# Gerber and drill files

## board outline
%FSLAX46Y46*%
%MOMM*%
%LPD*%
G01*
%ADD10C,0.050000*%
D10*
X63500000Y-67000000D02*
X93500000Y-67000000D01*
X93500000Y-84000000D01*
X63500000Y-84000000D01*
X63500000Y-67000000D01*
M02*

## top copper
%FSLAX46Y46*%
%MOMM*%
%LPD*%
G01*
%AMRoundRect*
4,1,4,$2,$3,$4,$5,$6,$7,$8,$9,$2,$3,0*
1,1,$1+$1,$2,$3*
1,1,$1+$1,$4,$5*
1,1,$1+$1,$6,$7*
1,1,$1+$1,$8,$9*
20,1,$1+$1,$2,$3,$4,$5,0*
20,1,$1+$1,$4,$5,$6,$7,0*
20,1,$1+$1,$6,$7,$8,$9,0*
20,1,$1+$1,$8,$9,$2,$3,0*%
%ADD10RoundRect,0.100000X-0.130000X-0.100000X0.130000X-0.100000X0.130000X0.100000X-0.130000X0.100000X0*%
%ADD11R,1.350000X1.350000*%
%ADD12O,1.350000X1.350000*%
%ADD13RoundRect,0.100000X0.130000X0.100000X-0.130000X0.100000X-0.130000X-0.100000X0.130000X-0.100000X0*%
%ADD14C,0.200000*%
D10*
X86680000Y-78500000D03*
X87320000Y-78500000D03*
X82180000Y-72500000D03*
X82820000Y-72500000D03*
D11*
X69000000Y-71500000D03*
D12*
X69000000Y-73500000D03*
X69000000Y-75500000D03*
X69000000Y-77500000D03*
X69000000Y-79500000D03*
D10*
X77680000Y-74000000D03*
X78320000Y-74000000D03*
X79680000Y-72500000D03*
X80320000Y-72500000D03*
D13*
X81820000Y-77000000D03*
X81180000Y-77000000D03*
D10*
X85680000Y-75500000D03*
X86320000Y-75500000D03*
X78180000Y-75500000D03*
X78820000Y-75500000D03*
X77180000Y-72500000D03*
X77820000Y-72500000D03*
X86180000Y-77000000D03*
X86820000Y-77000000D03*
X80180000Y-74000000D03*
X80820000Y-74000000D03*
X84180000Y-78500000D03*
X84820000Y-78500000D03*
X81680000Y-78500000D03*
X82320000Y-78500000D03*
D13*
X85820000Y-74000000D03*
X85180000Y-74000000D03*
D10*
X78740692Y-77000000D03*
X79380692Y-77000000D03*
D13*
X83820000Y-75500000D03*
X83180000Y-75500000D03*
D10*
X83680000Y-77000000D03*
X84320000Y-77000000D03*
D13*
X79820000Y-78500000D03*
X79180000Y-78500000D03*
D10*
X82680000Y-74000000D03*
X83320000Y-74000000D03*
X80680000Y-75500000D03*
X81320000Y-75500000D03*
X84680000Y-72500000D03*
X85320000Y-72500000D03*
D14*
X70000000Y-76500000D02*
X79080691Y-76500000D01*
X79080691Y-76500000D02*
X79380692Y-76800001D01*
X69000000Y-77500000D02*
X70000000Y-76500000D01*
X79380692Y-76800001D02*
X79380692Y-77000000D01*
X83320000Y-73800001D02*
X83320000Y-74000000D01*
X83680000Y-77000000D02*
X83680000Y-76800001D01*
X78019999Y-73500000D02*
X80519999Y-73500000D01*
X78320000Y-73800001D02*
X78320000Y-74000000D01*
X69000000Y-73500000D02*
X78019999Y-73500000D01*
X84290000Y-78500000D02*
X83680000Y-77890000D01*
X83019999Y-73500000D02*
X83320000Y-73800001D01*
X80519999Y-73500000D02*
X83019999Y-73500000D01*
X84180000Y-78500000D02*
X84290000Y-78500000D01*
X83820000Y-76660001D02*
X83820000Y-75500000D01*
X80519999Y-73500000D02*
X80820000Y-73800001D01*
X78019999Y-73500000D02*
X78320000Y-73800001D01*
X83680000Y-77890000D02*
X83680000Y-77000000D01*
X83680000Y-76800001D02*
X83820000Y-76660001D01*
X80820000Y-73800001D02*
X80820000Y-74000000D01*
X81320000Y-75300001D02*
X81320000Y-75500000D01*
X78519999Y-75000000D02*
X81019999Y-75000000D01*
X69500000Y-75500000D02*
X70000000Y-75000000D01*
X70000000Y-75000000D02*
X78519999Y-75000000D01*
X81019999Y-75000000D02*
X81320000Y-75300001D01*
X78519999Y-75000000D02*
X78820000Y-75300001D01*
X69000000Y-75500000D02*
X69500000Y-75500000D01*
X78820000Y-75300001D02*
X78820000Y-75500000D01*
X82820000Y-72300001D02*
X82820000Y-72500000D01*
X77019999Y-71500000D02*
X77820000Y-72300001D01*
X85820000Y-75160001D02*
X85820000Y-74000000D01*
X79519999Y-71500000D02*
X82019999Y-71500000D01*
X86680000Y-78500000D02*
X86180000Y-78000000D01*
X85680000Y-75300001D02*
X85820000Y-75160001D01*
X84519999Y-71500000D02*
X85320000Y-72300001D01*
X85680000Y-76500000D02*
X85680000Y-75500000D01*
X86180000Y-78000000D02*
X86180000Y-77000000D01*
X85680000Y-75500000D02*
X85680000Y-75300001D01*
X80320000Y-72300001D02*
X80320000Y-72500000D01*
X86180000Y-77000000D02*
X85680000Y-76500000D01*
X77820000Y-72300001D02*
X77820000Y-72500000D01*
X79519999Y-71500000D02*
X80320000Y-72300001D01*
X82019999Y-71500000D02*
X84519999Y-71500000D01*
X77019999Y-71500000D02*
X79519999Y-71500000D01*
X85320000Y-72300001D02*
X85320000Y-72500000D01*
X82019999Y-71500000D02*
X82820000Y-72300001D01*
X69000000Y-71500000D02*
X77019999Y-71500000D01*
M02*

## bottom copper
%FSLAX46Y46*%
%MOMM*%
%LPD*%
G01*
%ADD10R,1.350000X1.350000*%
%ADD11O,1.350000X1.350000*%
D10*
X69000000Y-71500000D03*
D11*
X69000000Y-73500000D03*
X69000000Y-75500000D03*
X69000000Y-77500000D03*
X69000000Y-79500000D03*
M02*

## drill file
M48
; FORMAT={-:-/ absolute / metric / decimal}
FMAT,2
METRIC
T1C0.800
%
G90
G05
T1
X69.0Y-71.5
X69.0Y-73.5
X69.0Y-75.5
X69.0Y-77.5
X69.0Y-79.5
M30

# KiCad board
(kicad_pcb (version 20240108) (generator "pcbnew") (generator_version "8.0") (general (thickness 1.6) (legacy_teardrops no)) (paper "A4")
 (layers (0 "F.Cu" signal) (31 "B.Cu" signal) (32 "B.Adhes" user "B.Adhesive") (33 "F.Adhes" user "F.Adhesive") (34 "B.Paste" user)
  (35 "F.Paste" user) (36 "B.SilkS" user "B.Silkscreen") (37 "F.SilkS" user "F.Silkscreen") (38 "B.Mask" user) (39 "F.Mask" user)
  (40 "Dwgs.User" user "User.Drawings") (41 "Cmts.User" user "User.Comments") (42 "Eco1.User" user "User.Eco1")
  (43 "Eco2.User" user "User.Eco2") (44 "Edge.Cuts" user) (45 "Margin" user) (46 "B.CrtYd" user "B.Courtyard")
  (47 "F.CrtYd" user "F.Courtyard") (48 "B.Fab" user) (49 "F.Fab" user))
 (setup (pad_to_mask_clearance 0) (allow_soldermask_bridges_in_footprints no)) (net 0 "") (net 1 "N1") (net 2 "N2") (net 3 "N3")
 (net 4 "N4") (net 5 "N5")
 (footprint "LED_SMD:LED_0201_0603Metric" (layer "F.Cu") (at 87 78.5)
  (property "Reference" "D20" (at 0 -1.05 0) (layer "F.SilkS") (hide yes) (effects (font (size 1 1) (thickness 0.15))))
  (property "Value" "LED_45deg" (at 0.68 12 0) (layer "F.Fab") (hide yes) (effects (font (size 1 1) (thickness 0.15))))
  (pad "" smd roundrect (at -0.345 0) (size 0.318 0.36) (layers "F.Paste") (roundrect_rratio 0.25))
  (pad "" smd roundrect (at 0.345 0) (size 0.318 0.36) (layers "F.Paste") (roundrect_rratio 0.25))
  (pad "1" smd roundrect (at -0.32 0) (size 0.46 0.4) (layers "F.Cu" "F.Mask") (roundrect_rratio 0.25) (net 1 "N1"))
  (pad "2" smd roundrect (at 0.32 0) (size 0.46 0.4) (layers "F.Cu" "F.Mask") (roundrect_rratio 0.25) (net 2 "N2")))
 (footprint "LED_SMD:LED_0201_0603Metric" (layer "F.Cu") (at 82.5 72.5)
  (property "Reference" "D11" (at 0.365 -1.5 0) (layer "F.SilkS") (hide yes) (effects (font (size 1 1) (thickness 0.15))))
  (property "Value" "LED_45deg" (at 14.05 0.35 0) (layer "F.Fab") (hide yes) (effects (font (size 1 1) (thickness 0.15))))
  (pad "" smd roundrect (at -0.345 0) (size 0.318 0.36) (layers "F.Paste") (roundrect_rratio 0.25))
  (pad "" smd roundrect (at 0.345 0) (size 0.318 0.36) (layers "F.Paste") (roundrect_rratio 0.25))
  (pad "1" smd roundrect (at -0.32 0) (size 0.46 0.4) (layers "F.Cu" "F.Mask") (roundrect_rratio 0.25) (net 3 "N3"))
  (pad "2" smd roundrect (at 0.32 0) (size 0.46 0.4) (layers "F.Cu" "F.Mask") (roundrect_rratio 0.25) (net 1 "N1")))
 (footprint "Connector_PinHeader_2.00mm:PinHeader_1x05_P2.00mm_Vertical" (layer "F.Cu") (at 69 71.5)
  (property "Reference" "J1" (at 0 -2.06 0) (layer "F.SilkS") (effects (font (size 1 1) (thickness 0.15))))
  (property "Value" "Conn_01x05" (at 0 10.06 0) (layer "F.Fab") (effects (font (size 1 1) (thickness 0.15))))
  (pad "1" thru_hole rect (at 0 0) (size 1.35 1.35) (drill 0.8) (layers "*.Cu" "*.Mask") (remove_unused_layers no) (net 1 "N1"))
  (pad "2" thru_hole oval (at 0 2) (size 1.35 1.35) (drill 0.8) (layers "*.Cu" "*.Mask") (remove_unused_layers no) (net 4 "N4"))
  (pad "3" thru_hole oval (at 0 4) (size 1.35 1.35) (drill 0.8) (layers "*.Cu" "*.Mask") (remove_unused_layers no) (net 3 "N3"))
  (pad "4" thru_hole oval (at 0 6) (size 1.35 1.35) (drill 0.8) (layers "*.Cu" "*.Mask") (remove_unused_layers no) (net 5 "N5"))
  (pad "5" thru_hole oval (at 0 8) (size 1.35 1.35) (drill 0.8) (layers "*.Cu" "*.Mask") (remove_unused_layers no) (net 2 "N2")))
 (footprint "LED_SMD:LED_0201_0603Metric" (layer "F.Cu") (at 78 74)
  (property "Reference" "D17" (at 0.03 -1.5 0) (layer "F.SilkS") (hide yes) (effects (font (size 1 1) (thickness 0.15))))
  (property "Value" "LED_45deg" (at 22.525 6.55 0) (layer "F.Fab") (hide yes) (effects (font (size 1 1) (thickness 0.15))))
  (pad "" smd roundrect (at -0.345 0) (size 0.318 0.36) (layers "F.Paste") (roundrect_rratio 0.25))
  (pad "" smd roundrect (at 0.345 0) (size 0.318 0.36) (layers "F.Paste") (roundrect_rratio 0.25))
  (pad "1" smd roundrect (at -0.32 0) (size 0.46 0.4) (layers "F.Cu" "F.Mask") (roundrect_rratio 0.25) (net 2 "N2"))
  (pad "2" smd roundrect (at 0.32 0) (size 0.46 0.4) (layers "F.Cu" "F.Mask") (roundrect_rratio 0.25) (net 4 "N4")))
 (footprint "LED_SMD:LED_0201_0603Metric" (layer "F.Cu") (at 80 72.5)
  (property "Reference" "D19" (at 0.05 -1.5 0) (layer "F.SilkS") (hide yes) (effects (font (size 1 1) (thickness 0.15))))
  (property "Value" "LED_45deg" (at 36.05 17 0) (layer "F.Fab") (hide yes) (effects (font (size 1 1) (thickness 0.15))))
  (pad "" smd roundrect (at -0.345 0) (size 0.318 0.36) (layers "F.Paste") (roundrect_rratio 0.25))
  (pad "" smd roundrect (at 0.345 0) (size 0.318 0.36) (layers "F.Paste") (roundrect_rratio 0.25))
  (pad "1" smd roundrect (at -0.32 0) (size 0.46 0.4) (layers "F.Cu" "F.Mask") (roundrect_rratio 0.25) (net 5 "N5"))
  (pad "2" smd roundrect (at 0.32 0) (size 0.46 0.4) (layers "F.Cu" "F.Mask") (roundrect_rratio 0.25) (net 1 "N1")))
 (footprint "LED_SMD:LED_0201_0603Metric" (layer "F.Cu") (at 81.5 77 180)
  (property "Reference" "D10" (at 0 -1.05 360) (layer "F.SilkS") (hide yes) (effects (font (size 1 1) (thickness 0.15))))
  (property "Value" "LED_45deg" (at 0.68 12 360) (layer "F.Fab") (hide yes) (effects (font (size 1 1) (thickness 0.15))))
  (pad "" smd roundrect (at -0.345 0 180) (size 0.318 0.36) (layers "F.Paste") (roundrect_rratio 0.25))
  (pad "" smd roundrect (at 0.345 0 180) (size 0.318 0.36) (layers "F.Paste") (roundrect_rratio 0.25))
  (pad "1" smd roundrect (at -0.32 0 180) (size 0.46 0.4) (layers "F.Cu" "F.Mask") (roundrect_rratio 0.25) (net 3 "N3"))
  (pad "2" smd roundrect (at 0.32 0 180) (size 0.46 0.4) (layers "F.Cu" "F.Mask") (roundrect_rratio 0.25) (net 5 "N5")))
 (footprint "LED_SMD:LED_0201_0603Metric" (layer "F.Cu") (at 86 75.5)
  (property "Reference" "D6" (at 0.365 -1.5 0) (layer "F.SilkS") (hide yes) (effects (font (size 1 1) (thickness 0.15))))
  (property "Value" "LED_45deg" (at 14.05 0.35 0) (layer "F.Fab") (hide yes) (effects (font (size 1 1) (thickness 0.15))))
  (pad "" smd roundrect (at -0.345 0) (size 0.318 0.36) (layers "F.Paste") (roundrect_rratio 0.25))
  (pad "" smd roundrect (at 0.345 0) (size 0.318 0.36) (layers "F.Paste") (roundrect_rratio 0.25))
  (pad "1" smd roundrect (at -0.32 0) (size 0.46 0.4) (layers "F.Cu" "F.Mask") (roundrect_rratio 0.25) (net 1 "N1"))
  (pad "2" smd roundrect (at 0.32 0) (size 0.46 0.4) (layers "F.Cu" "F.Mask") (roundrect_rratio 0.25) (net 3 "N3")))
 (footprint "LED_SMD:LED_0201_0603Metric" (layer "F.Cu") (at 78.5 75.5)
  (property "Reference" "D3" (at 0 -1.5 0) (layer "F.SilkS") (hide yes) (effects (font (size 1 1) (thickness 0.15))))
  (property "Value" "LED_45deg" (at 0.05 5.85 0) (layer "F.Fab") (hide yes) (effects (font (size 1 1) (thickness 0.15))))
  (pad "" smd roundrect (at -0.345 0) (size 0.318 0.36) (layers "F.Paste") (roundrect_rratio 0.25))
  (pad "" smd roundrect (at 0.345 0) (size 0.318 0.36) (layers "F.Paste") (roundrect_rratio 0.25))
  (pad "1" smd roundrect (at -0.32 0) (size 0.46 0.4) (layers "F.Cu" "F.Mask") (roundrect_rratio 0.25) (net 2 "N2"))
  (pad "2" smd roundrect (at 0.32 0) (size 0.46 0.4) (layers "F.Cu" "F.Mask") (roundrect_rratio 0.25) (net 3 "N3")))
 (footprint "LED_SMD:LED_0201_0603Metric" (layer "F.Cu") (at 77.5 72.5)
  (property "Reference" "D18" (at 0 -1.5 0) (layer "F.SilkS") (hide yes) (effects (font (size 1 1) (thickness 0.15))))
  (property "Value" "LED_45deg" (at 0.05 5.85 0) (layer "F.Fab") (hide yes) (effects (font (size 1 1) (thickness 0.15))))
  (pad "" smd roundrect (at -0.345 0) (size 0.318 0.36) (layers "F.Paste") (roundrect_rratio 0.25))
  (pad "" smd roundrect (at 0.345 0) (size 0.318 0.36) (layers "F.Paste") (roundrect_rratio 0.25))
  (pad "1" smd roundrect (at -0.32 0) (size 0.46 0.4) (layers "F.Cu" "F.Mask") (roundrect_rratio 0.25) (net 2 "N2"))
  (pad "2" smd roundrect (at 0.32 0) (size 0.46 0.4) (layers "F.Cu" "F.Mask") (roundrect_rratio 0.25) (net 1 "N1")))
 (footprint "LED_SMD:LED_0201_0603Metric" (layer "F.Cu") (at 86.5 77)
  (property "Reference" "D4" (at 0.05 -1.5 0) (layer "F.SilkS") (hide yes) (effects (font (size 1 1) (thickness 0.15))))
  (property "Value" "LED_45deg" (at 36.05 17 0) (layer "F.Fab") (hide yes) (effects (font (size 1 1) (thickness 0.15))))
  (pad "" smd roundrect (at -0.345 0) (size 0.318 0.36) (layers "F.Paste") (roundrect_rratio 0.25))
  (pad "" smd roundrect (at 0.345 0) (size 0.318 0.36) (layers "F.Paste") (roundrect_rratio 0.25))
  (pad "1" smd roundrect (at -0.32 0) (size 0.46 0.4) (layers "F.Cu" "F.Mask") (roundrect_rratio 0.25) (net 1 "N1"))
  (pad "2" smd roundrect (at 0.32 0) (size 0.46 0.4) (layers "F.Cu" "F.Mask") (roundrect_rratio 0.25) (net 5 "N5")))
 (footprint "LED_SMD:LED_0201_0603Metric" (layer "F.Cu") (at 80.5 74)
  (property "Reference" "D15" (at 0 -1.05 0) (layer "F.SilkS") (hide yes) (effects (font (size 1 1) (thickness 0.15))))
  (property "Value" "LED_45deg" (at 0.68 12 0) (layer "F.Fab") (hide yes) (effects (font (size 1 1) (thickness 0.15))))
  (pad "" smd roundrect (at -0.345 0) (size 0.318 0.36) (layers "F.Paste") (roundrect_rratio 0.25))
  (pad "" smd roundrect (at 0.345 0) (size 0.318 0.36) (layers "F.Paste") (roundrect_rratio 0.25))
  (pad "1" smd roundrect (at -0.32 0) (size 0.46 0.4) (layers "F.Cu" "F.Mask") (roundrect_rratio 0.25) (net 5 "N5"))
  (pad "2" smd roundrect (at 0.32 0) (size 0.46 0.4) (layers "F.Cu" "F.Mask") (roundrect_rratio 0.25) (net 4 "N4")))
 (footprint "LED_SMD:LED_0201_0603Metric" (layer "F.Cu") (at 84.5 78.5)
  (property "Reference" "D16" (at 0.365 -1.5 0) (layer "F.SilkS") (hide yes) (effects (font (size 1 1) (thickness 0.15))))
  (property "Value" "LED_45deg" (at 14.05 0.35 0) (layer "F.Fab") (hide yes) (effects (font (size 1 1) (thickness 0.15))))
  (pad "" smd roundrect (at -0.345 0) (size 0.318 0.36) (layers "F.Paste") (roundrect_rratio 0.25))
  (pad "" smd roundrect (at 0.345 0) (size 0.318 0.36) (layers "F.Paste") (roundrect_rratio 0.25))
  (pad "1" smd roundrect (at -0.32 0) (size 0.46 0.4) (layers "F.Cu" "F.Mask") (roundrect_rratio 0.25) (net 4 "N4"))
  (pad "2" smd roundrect (at 0.32 0) (size 0.46 0.4) (layers "F.Cu" "F.Mask") (roundrect_rratio 0.25) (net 2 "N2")))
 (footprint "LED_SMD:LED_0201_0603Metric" (layer "F.Cu") (at 82 78.5)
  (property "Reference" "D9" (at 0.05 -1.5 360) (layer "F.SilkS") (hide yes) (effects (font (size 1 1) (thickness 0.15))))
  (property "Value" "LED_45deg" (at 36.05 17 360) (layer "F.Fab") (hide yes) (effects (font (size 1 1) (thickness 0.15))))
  (pad "" smd roundrect (at -0.345 0) (size 0.318 0.36) (layers "F.Paste") (roundrect_rratio 0.25))
  (pad "" smd roundrect (at 0.345 0) (size 0.318 0.36) (layers "F.Paste") (roundrect_rratio 0.25))
  (pad "1" smd roundrect (at -0.32 0) (size 0.46 0.4) (layers "F.Cu" "F.Mask") (roundrect_rratio 0.25) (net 3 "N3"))
  (pad "2" smd roundrect (at 0.32 0) (size 0.46 0.4) (layers "F.Cu" "F.Mask") (roundrect_rratio 0.25) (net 2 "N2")))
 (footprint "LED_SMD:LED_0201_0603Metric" (layer "F.Cu") (at 85.5 74 180)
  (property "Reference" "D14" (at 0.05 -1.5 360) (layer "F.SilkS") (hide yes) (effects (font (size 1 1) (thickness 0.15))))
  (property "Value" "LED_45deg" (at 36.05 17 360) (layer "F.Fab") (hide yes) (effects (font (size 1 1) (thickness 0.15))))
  (pad "" smd roundrect (at -0.345 0 180) (size 0.318 0.36) (layers "F.Paste") (roundrect_rratio 0.25))
  (pad "" smd roundrect (at 0.345 0 180) (size 0.318 0.36) (layers "F.Paste") (roundrect_rratio 0.25))
  (pad "1" smd roundrect (at -0.32 0 180) (size 0.46 0.4) (layers "F.Cu" "F.Mask") (roundrect_rratio 0.25) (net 1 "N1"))
  (pad "2" smd roundrect (at 0.32 0 180) (size 0.46 0.4) (layers "F.Cu" "F.Mask") (roundrect_rratio 0.25) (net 4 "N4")))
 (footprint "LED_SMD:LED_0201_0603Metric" (layer "F.Cu") (at 79.060692 77)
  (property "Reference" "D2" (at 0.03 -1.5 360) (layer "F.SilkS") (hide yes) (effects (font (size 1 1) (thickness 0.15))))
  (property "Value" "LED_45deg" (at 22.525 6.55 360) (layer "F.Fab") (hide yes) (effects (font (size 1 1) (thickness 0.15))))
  (pad "" smd roundrect (at -0.345 0) (size 0.318 0.36) (layers "F.Paste") (roundrect_rratio 0.25))
  (pad "" smd roundrect (at 0.345 0) (size 0.318 0.36) (layers "F.Paste") (roundrect_rratio 0.25))
  (pad "1" smd roundrect (at -0.32 0) (size 0.46 0.4) (layers "F.Cu" "F.Mask") (roundrect_rratio 0.25) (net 2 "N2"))
  (pad "2" smd roundrect (at 0.32 0) (size 0.46 0.4) (layers "F.Cu" "F.Mask") (roundrect_rratio 0.25) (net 5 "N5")))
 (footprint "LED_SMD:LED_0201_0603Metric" (layer "F.Cu") (at 83.5 75.5 180)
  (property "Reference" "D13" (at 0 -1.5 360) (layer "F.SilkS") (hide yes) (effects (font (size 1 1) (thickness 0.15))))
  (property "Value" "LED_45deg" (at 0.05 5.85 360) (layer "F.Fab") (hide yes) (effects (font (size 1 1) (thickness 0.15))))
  (pad "" smd roundrect (at -0.345 0 180) (size 0.318 0.36) (layers "F.Paste") (roundrect_rratio 0.25))
  (pad "" smd roundrect (at 0.345 0 180) (size 0.318 0.36) (layers "F.Paste") (roundrect_rratio 0.25))
  (pad "1" smd roundrect (at -0.32 0 180) (size 0.46 0.4) (layers "F.Cu" "F.Mask") (roundrect_rratio 0.25) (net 4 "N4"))
  (pad "2" smd roundrect (at 0.32 0 180) (size 0.46 0.4) (layers "F.Cu" "F.Mask") (roundrect_rratio 0.25) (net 3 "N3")))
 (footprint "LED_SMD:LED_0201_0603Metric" (layer "F.Cu") (at 84 77)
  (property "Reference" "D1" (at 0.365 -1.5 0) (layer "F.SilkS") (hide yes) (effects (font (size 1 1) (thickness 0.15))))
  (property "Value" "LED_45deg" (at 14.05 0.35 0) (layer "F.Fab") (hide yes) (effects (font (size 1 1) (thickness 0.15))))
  (pad "" smd roundrect (at -0.345 0) (size 0.318 0.36) (layers "F.Paste") (roundrect_rratio 0.25))
  (pad "" smd roundrect (at 0.345 0) (size 0.318 0.36) (layers "F.Paste") (roundrect_rratio 0.25))
  (pad "1" smd roundrect (at -0.32 0) (size 0.46 0.4) (layers "F.Cu" "F.Mask") (roundrect_rratio 0.25) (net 4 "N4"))
  (pad "2" smd roundrect (at 0.32 0) (size 0.46 0.4) (layers "F.Cu" "F.Mask") (roundrect_rratio 0.25) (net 5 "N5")))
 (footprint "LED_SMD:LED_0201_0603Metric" (layer "F.Cu") (at 79.5 78.5 180)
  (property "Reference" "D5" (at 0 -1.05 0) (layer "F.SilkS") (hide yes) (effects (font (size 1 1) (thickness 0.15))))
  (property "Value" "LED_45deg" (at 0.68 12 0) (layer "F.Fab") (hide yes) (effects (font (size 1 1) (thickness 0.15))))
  (pad "" smd roundrect (at -0.345 0 180) (size 0.318 0.36) (layers "F.Paste") (roundrect_rratio 0.25))
  (pad "" smd roundrect (at 0.345 0 180) (size 0.318 0.36) (layers "F.Paste") (roundrect_rratio 0.25))
  (pad "1" smd roundrect (at -0.32 0 180) (size 0.46 0.4) (layers "F.Cu" "F.Mask") (roundrect_rratio 0.25) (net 5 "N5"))
  (pad "2" smd roundrect (at 0.32 0 180) (size 0.46 0.4) (layers "F.Cu" "F.Mask") (roundrect_rratio 0.25) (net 2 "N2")))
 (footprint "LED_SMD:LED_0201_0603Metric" (layer "F.Cu") (at 83 74)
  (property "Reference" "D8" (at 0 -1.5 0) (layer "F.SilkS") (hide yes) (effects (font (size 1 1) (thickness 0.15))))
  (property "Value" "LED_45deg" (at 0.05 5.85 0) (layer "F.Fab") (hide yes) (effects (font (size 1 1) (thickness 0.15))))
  (pad "" smd roundrect (at -0.345 0) (size 0.318 0.36) (layers "F.Paste") (roundrect_rratio 0.25))
  (pad "" smd roundrect (at 0.345 0) (size 0.318 0.36) (layers "F.Paste") (roundrect_rratio 0.25))
  (pad "1" smd roundrect (at -0.32 0) (size 0.46 0.4) (layers "F.Cu" "F.Mask") (roundrect_rratio 0.25) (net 3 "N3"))
  (pad "2" smd roundrect (at 0.32 0) (size 0.46 0.4) (layers "F.Cu" "F.Mask") (roundrect_rratio 0.25) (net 4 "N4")))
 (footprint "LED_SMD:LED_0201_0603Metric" (layer "F.Cu") (at 81 75.5)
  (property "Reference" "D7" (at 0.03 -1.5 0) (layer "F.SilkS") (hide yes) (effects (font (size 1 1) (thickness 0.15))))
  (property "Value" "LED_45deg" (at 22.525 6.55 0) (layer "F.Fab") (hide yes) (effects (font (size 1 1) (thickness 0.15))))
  (pad "" smd roundrect (at -0.345 0) (size 0.318 0.36) (layers "F.Paste") (roundrect_rratio 0.25))
  (pad "" smd roundrect (at 0.345 0) (size 0.318 0.36) (layers "F.Paste") (roundrect_rratio 0.25))
  (pad "1" smd roundrect (at -0.32 0) (size 0.46 0.4) (layers "F.Cu" "F.Mask") (roundrect_rratio 0.25) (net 5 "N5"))
  (pad "2" smd roundrect (at 0.32 0) (size 0.46 0.4) (layers "F.Cu" "F.Mask") (roundrect_rratio 0.25) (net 3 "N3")))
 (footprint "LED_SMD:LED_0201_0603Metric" (layer "F.Cu") (at 85 72.5)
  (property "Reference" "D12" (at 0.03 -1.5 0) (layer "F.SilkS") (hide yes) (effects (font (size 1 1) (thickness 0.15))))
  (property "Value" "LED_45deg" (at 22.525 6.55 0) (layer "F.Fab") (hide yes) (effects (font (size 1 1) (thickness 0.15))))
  (pad "" smd roundrect (at -0.345 0) (size 0.318 0.36) (layers "F.Paste") (roundrect_rratio 0.25))
  (pad "" smd roundrect (at 0.345 0) (size 0.318 0.36) (layers "F.Paste") (roundrect_rratio 0.25))
  (pad "1" smd roundrect (at -0.32 0) (size 0.46 0.4) (layers "F.Cu" "F.Mask") (roundrect_rratio 0.25) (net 4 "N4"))
  (pad "2" smd roundrect (at 0.32 0) (size 0.46 0.4) (layers "F.Cu" "F.Mask") (roundrect_rratio 0.25) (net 1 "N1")))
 (gr_rect (start 63.5 67) (end 93.5 84) (stroke (width 0.05) (type default)) (fill none) (layer "Edge.Cuts"))
 (segment (start 70 76.5) (end 79.080691 76.5) (width 0.2) (layer "F.Cu") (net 5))
 (segment (start 79.080691 76.5) (end 79.380692 76.800001) (width 0.2) (layer "F.Cu") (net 5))
 (segment (start 69 77.5) (end 70 76.5) (width 0.2) (layer "F.Cu") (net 5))
 (segment (start 79.380692 76.800001) (end 79.380692 77) (width 0.2) (layer "F.Cu") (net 5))
 (segment (start 83.32 73.800001) (end 83.32 74) (width 0.2) (layer "F.Cu") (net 4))
 (segment (start 83.68 77) (end 83.68 76.800001) (width 0.2) (layer "F.Cu") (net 4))
 (segment (start 78.019999 73.5) (end 80.519999 73.5) (width 0.2) (layer "F.Cu") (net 4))
 (segment (start 78.32 73.800001) (end 78.32 74) (width 0.2) (layer "F.Cu") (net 4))
 (segment (start 69 73.5) (end 78.019999 73.5) (width 0.2) (layer "F.Cu") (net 4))
 (segment (start 84.29 78.5) (end 83.68 77.89) (width 0.2) (layer "F.Cu") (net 4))
 (segment (start 83.019999 73.5) (end 83.32 73.800001) (width 0.2) (layer "F.Cu") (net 4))
 (segment (start 80.519999 73.5) (end 83.019999 73.5) (width 0.2) (layer "F.Cu") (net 4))
 (segment (start 84.18 78.5) (end 84.29 78.5) (width 0.2) (layer "F.Cu") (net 4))
 (segment (start 83.82 76.660001) (end 83.82 75.5) (width 0.2) (layer "F.Cu") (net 4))
 (segment (start 80.519999 73.5) (end 80.82 73.800001) (width 0.2) (layer "F.Cu") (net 4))
 (segment (start 78.019999 73.5) (end 78.32 73.800001) (width 0.2) (layer "F.Cu") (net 4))
 (segment (start 83.68 77.89) (end 83.68 77) (width 0.2) (layer "F.Cu") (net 4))
 (segment (start 83.68 76.800001) (end 83.82 76.660001) (width 0.2) (layer "F.Cu") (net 4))
 (segment (start 80.82 73.800001) (end 80.82 74) (width 0.2) (layer "F.Cu") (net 4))
 (segment (start 81.32 75.300001) (end 81.32 75.5) (width 0.2) (layer "F.Cu") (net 3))
 (segment (start 78.519999 75) (end 81.019999 75) (width 0.2) (layer "F.Cu") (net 3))
 (segment (start 69.5 75.5) (end 70 75) (width 0.2) (layer "F.Cu") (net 3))
 (segment (start 70 75) (end 78.519999 75) (width 0.2) (layer "F.Cu") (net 3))
 (segment (start 81.019999 75) (end 81.32 75.300001) (width 0.2) (layer "F.Cu") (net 3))
 (segment (start 78.519999 75) (end 78.82 75.300001) (width 0.2) (layer "F.Cu") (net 3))
 (segment (start 69 75.5) (end 69.5 75.5) (width 0.2) (layer "F.Cu") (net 3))
 (segment (start 78.82 75.300001) (end 78.82 75.5) (width 0.2) (layer "F.Cu") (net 3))
 (segment (start 82.82 72.300001) (end 82.82 72.5) (width 0.2) (layer "F.Cu") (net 1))
 (segment (start 77.019999 71.5) (end 77.82 72.300001) (width 0.2) (layer "F.Cu") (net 1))
 (segment (start 85.82 75.160001) (end 85.82 74) (width 0.2) (layer "F.Cu") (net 1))
 (segment (start 79.519999 71.5) (end 82.019999 71.5) (width 0.2) (layer "F.Cu") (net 1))
 (segment (start 86.68 78.5) (end 86.18 78) (width 0.2) (layer "F.Cu") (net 1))
 (segment (start 85.68 75.300001) (end 85.82 75.160001) (width 0.2) (layer "F.Cu") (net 1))
 (segment (start 84.519999 71.5) (end 85.32 72.300001) (width 0.2) (layer "F.Cu") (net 1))
 (segment (start 85.68 76.5) (end 85.68 75.5) (width 0.2) (layer "F.Cu") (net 1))
 (segment (start 86.18 78) (end 86.18 77) (width 0.2) (layer "F.Cu") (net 1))
 (segment (start 85.68 75.5) (end 85.68 75.300001) (width 0.2) (layer "F.Cu") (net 1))
 (segment (start 80.32 72.300001) (end 80.32 72.5) (width 0.2) (layer "F.Cu") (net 1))
 (segment (start 86.18 77) (end 85.68 76.5) (width 0.2) (layer "F.Cu") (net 1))
 (segment (start 77.82 72.300001) (end 77.82 72.5) (width 0.2) (layer "F.Cu") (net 1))
 (segment (start 79.519999 71.5) (end 80.32 72.300001) (width 0.2) (layer "F.Cu") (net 1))
 (segment (start 82.019999 71.5) (end 84.519999 71.5) (width 0.2) (layer "F.Cu") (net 1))
 (segment (start 77.019999 71.5) (end 79.519999 71.5) (width 0.2) (layer "F.Cu") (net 1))
 (segment (start 85.32 72.300001) (end 85.32 72.5) (width 0.2) (layer "F.Cu") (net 1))
 (segment (start 82.019999 71.5) (end 82.82 72.300001) (width 0.2) (layer "F.Cu") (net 1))
 (segment (start 69 71.5) (end 77.019999 71.5) (width 0.2) (layer "F.Cu") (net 1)))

